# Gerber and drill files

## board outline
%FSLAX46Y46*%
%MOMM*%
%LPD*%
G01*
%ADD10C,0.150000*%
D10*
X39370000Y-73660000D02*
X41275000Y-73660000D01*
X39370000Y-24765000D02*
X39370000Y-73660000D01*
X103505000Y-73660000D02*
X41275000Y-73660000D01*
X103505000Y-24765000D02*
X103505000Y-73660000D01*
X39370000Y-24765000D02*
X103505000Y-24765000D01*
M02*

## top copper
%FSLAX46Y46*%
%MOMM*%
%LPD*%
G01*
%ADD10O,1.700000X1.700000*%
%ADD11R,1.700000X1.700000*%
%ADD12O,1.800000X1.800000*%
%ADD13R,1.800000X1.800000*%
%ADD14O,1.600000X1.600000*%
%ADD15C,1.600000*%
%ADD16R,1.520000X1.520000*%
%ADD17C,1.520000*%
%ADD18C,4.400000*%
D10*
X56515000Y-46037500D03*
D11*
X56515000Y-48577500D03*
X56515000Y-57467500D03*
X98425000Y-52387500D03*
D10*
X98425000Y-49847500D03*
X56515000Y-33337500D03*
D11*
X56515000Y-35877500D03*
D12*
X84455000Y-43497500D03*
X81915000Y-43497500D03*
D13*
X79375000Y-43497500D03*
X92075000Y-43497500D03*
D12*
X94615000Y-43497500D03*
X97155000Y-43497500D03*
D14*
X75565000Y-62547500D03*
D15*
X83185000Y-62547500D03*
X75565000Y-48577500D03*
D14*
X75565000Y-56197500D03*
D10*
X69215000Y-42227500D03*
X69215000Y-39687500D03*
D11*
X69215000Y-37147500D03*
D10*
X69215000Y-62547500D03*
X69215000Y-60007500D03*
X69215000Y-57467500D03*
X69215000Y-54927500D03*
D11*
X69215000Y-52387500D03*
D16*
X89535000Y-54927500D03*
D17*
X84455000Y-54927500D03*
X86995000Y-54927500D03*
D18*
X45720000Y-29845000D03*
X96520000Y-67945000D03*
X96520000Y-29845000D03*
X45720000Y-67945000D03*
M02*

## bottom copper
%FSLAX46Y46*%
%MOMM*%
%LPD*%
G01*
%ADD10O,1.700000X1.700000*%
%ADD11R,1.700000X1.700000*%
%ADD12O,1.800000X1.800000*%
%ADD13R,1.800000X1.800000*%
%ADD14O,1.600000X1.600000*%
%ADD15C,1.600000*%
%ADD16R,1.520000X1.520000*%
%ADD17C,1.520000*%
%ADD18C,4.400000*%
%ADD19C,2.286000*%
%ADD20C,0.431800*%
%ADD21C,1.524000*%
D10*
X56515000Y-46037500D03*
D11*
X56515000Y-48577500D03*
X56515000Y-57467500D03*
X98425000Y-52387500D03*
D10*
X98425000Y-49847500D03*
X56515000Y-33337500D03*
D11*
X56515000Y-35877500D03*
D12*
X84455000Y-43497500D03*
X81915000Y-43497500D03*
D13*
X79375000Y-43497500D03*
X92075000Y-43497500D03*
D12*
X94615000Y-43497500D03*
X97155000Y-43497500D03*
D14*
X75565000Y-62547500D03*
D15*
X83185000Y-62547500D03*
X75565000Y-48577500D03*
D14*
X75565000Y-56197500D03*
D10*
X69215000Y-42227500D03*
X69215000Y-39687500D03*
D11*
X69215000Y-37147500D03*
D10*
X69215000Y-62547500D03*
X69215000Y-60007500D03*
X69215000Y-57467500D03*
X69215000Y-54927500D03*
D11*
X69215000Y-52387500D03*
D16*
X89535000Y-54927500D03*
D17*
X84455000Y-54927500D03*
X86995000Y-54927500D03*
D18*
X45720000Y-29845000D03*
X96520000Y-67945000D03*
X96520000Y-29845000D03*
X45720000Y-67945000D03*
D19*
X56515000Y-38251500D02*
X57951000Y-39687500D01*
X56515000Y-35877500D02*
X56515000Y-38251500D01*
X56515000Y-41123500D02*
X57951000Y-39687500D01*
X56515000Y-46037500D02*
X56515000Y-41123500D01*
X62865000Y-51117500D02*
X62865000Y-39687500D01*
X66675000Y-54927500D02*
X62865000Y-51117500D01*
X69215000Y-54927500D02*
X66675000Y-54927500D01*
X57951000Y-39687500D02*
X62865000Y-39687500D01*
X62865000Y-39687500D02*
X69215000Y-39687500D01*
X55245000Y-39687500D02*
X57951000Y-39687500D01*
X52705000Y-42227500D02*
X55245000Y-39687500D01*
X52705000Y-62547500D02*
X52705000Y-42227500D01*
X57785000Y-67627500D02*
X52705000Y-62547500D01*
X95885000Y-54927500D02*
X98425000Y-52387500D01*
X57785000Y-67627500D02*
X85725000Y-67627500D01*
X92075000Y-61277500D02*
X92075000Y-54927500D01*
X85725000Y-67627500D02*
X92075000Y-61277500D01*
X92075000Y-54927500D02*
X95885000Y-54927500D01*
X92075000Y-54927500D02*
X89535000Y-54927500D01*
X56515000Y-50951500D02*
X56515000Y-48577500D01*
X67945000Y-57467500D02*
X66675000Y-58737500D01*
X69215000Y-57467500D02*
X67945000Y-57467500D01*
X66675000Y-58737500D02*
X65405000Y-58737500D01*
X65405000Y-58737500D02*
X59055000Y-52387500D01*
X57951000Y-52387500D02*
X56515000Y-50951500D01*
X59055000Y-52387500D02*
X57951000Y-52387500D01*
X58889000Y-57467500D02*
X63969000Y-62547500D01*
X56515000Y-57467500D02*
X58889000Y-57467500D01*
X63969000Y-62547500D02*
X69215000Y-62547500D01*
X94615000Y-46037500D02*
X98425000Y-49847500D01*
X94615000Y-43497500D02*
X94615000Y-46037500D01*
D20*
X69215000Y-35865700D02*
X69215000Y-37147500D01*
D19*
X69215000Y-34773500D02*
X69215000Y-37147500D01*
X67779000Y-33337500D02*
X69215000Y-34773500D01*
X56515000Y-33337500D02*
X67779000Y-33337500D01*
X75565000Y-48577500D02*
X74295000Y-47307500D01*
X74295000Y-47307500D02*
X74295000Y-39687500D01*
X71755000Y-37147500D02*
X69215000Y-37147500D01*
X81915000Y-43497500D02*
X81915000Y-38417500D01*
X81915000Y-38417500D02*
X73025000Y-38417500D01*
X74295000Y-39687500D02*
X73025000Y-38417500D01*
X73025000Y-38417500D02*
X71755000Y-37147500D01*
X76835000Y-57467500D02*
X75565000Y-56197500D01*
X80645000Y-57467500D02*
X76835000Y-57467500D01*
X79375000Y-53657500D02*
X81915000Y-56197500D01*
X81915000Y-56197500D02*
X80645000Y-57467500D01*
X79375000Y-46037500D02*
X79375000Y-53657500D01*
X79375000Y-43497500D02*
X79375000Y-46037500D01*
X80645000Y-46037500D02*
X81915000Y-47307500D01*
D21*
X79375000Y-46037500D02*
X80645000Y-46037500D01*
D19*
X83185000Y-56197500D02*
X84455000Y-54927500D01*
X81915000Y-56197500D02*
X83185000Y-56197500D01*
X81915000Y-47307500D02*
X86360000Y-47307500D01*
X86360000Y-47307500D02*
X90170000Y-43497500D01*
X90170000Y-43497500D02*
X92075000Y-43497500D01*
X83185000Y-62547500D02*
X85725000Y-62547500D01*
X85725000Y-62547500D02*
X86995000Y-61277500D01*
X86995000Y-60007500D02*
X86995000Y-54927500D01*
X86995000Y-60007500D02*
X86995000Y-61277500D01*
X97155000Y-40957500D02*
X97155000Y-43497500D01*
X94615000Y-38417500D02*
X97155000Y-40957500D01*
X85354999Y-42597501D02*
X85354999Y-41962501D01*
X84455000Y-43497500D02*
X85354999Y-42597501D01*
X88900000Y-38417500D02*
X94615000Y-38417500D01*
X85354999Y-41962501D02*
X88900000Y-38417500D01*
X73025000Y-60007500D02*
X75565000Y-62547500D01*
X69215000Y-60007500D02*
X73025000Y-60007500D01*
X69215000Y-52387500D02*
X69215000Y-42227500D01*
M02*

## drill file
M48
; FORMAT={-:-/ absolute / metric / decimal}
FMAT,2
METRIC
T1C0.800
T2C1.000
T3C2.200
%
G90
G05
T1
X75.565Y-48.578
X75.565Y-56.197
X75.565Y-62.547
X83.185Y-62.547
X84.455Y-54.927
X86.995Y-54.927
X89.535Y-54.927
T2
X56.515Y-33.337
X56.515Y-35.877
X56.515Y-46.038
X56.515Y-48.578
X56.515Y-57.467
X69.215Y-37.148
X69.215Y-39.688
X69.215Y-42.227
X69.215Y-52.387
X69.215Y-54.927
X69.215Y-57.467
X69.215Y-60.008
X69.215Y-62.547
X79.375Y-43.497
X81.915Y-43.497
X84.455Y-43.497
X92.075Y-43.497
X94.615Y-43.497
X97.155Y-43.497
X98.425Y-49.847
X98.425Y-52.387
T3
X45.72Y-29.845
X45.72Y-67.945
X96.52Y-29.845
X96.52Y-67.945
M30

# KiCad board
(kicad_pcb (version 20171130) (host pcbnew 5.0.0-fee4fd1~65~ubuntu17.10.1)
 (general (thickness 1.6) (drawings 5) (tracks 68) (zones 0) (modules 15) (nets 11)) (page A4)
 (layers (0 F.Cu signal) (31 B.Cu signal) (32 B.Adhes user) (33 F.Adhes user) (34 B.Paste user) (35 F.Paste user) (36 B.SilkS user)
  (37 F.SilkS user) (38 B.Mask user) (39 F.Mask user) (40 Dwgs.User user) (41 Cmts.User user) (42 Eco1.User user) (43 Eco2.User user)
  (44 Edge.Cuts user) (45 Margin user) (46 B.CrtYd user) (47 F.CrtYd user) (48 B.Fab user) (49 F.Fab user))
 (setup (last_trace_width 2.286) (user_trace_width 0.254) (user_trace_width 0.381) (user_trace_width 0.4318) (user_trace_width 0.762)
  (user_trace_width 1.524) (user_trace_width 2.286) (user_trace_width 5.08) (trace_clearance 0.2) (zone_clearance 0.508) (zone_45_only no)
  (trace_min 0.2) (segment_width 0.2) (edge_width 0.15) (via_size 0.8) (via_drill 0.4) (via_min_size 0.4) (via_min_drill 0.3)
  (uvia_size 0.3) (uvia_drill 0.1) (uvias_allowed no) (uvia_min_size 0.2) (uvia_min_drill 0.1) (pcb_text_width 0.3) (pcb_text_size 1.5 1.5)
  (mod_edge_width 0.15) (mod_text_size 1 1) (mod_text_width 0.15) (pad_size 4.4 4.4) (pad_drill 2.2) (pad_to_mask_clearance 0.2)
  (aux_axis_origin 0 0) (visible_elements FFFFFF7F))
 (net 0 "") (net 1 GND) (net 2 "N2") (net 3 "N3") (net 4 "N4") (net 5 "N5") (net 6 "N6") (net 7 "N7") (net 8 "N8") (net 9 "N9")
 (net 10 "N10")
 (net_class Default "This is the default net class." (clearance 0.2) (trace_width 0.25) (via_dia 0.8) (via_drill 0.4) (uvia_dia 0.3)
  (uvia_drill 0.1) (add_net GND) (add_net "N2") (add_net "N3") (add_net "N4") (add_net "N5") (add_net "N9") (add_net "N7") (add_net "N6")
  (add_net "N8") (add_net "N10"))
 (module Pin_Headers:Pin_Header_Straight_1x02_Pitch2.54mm (layer F.Cu) (at 56.515 48.5775 180)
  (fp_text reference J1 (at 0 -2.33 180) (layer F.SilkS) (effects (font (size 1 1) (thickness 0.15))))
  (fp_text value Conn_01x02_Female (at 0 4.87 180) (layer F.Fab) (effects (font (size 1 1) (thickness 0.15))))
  (pad 2 thru_hole oval (at 0 2.54 180) (size 1.7 1.7) (drill 1) (layers *.Cu *.Mask) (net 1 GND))
  (pad 1 thru_hole rect (at 0 0 180) (size 1.7 1.7) (drill 1) (layers *.Cu *.Mask) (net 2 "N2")))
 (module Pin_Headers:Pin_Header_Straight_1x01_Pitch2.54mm (layer F.Cu) (at 56.515 57.4675)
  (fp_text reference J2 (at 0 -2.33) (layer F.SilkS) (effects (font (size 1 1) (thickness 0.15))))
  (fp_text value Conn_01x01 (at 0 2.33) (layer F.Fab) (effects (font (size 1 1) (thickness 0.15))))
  (pad 1 thru_hole rect (at 0 0) (size 1.7 1.7) (drill 1) (layers *.Cu *.Mask) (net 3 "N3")))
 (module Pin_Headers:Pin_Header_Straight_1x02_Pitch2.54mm (layer F.Cu) (at 98.425 52.3875 180)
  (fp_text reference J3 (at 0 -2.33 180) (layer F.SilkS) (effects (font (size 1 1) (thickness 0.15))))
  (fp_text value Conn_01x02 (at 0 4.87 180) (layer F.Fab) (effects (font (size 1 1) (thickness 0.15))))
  (pad 1 thru_hole rect (at 0 0 180) (size 1.7 1.7) (drill 1) (layers *.Cu *.Mask) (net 1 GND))
  (pad 2 thru_hole oval (at 0 2.54 180) (size 1.7 1.7) (drill 1) (layers *.Cu *.Mask) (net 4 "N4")))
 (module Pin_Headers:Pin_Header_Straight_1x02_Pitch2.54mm (layer F.Cu) (at 56.515 35.8775 180)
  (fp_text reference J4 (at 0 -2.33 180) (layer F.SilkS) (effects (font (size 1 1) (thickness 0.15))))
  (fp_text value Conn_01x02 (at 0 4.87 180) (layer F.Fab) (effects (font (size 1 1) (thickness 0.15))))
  (pad 2 thru_hole oval (at 0 2.54 180) (size 1.7 1.7) (drill 1) (layers *.Cu *.Mask) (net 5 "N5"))
  (pad 1 thru_hole rect (at 0 0 180) (size 1.7 1.7) (drill 1) (layers *.Cu *.Mask) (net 1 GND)))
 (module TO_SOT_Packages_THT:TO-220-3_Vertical (layer F.Cu) (at 79.375 43.4975)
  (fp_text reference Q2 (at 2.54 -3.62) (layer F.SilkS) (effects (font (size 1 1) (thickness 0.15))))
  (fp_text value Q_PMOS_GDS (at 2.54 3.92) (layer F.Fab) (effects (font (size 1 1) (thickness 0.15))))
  (pad 3 thru_hole oval (at 5.08 0) (size 1.8 1.8) (drill 1) (layers *.Cu *.Mask) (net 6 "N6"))
  (pad 2 thru_hole oval (at 2.54 0) (size 1.8 1.8) (drill 1) (layers *.Cu *.Mask) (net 5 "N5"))
  (pad 1 thru_hole rect (at 0 0) (size 1.8 1.8) (drill 1) (layers *.Cu *.Mask) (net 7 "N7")))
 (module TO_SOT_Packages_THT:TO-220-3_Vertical (layer F.Cu) (at 92.075 43.4975)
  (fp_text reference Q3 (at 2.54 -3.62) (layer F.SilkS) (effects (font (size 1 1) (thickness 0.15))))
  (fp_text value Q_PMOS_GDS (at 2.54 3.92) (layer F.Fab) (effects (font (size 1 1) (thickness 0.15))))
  (pad 1 thru_hole rect (at 0 0) (size 1.8 1.8) (drill 1) (layers *.Cu *.Mask) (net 7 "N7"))
  (pad 2 thru_hole oval (at 2.54 0) (size 1.8 1.8) (drill 1) (layers *.Cu *.Mask) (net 4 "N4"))
  (pad 3 thru_hole oval (at 5.08 0) (size 1.8 1.8) (drill 1) (layers *.Cu *.Mask) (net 6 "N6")))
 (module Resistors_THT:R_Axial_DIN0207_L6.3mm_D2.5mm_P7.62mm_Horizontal (layer F.Cu) (at 83.185 62.5475 180)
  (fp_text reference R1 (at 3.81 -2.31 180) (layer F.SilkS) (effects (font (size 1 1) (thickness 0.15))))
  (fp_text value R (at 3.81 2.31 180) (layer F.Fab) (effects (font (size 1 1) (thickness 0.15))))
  (pad 2 thru_hole oval (at 7.62 0 180) (size 1.6 1.6) (drill 0.8) (layers *.Cu *.Mask) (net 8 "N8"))
  (pad 1 thru_hole circle (at 0 0 180) (size 1.6 1.6) (drill 0.8) (layers *.Cu *.Mask) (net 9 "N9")))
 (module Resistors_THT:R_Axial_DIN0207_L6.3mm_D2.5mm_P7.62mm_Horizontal (layer F.Cu) (at 75.565 48.5775 270)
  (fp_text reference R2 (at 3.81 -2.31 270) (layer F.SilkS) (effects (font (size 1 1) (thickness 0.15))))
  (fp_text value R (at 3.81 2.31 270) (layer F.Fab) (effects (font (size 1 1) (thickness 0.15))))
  (pad 1 thru_hole circle (at 0 0 270) (size 1.6 1.6) (drill 0.8) (layers *.Cu *.Mask) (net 5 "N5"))
  (pad 2 thru_hole oval (at 7.62 0 270) (size 1.6 1.6) (drill 0.8) (layers *.Cu *.Mask) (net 7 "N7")))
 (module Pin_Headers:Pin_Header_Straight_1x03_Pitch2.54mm (layer F.Cu) (at 69.215 37.1475)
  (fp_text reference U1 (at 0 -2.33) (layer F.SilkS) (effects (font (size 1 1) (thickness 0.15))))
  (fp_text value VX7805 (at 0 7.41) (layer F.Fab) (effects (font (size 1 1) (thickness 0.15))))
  (pad 3 thru_hole oval (at 0 5.08) (size 1.7 1.7) (drill 1) (layers *.Cu *.Mask) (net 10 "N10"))
  (pad 2 thru_hole oval (at 0 2.54) (size 1.7 1.7) (drill 1) (layers *.Cu *.Mask) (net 1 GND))
  (pad 1 thru_hole rect (at 0 0) (size 1.7 1.7) (drill 1) (layers *.Cu *.Mask) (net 5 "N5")))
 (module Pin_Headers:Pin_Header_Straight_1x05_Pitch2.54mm (layer F.Cu) (at 69.215 52.3875)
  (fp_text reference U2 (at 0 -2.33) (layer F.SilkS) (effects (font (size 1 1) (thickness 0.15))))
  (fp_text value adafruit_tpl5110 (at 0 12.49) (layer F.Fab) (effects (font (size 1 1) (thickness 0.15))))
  (pad 5 thru_hole oval (at 0 10.16) (size 1.7 1.7) (drill 1) (layers *.Cu *.Mask) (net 3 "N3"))
  (pad 4 thru_hole oval (at 0 7.62) (size 1.7 1.7) (drill 1) (layers *.Cu *.Mask) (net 8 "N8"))
  (pad 3 thru_hole oval (at 0 5.08) (size 1.7 1.7) (drill 1) (layers *.Cu *.Mask) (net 2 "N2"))
  (pad 2 thru_hole oval (at 0 2.54) (size 1.7 1.7) (drill 1) (layers *.Cu *.Mask) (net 1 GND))
  (pad 1 thru_hole rect (at 0 0) (size 1.7 1.7) (drill 1) (layers *.Cu *.Mask) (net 10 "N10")))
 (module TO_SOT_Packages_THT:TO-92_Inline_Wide (layer F.Cu) (at 89.535 54.9275 180)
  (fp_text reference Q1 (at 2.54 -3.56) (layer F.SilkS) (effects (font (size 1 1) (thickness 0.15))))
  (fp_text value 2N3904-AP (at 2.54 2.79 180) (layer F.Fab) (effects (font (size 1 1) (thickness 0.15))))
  (pad 1 thru_hole rect (at 0 0 270) (size 1.52 1.52) (drill 0.8) (layers *.Cu *.Mask) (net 1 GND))
  (pad 3 thru_hole circle (at 5.08 0 270) (size 1.52 1.52) (drill 0.8) (layers *.Cu *.Mask) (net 7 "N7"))
  (pad 2 thru_hole circle (at 2.54 0 270) (size 1.52 1.52) (drill 0.8) (layers *.Cu *.Mask) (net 9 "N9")))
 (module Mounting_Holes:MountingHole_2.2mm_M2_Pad (layer F.Cu) (at 45.72 29.845)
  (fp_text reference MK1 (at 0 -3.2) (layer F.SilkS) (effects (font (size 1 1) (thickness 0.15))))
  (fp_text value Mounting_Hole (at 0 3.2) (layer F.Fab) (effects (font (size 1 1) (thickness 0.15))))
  (pad 1 thru_hole circle (at 0 0) (size 4.4 4.4) (drill 2.2) (layers *.Cu *.Mask)))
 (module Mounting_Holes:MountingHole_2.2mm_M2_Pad (layer F.Cu) (at 96.52 67.945)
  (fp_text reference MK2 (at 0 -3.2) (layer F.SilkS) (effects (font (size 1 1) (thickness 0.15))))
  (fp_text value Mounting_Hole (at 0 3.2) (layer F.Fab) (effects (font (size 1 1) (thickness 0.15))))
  (pad 1 thru_hole circle (at 0 0) (size 4.4 4.4) (drill 2.2) (layers *.Cu *.Mask)))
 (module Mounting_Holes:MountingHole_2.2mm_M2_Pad (layer F.Cu) (at 96.52 29.845)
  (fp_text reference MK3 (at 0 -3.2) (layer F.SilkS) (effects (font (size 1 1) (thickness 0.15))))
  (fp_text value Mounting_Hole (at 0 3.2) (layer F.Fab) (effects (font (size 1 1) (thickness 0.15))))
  (pad 1 thru_hole circle (at 0 0) (size 4.4 4.4) (drill 2.2) (layers *.Cu *.Mask)))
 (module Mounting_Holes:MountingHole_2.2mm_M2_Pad (layer F.Cu) (at 45.72 67.945)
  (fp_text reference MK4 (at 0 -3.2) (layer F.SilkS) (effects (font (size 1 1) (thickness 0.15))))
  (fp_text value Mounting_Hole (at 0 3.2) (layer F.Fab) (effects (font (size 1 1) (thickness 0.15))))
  (pad 1 thru_hole circle (at 0 0) (size 4.4 4.4) (drill 2.2) (layers *.Cu *.Mask)))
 (gr_line (start 39.37 73.66) (end 41.275 73.66) (layer Edge.Cuts) (width 0.15))
 (gr_line (start 39.37 24.765) (end 39.37 73.66) (layer Edge.Cuts) (width 0.15))
 (gr_line (start 103.505 73.66) (end 41.275 73.66) (layer Edge.Cuts) (width 0.15))
 (gr_line (start 103.505 24.765) (end 103.505 73.66) (layer Edge.Cuts) (width 0.15))
 (gr_line (start 39.37 24.765) (end 103.505 24.765) (layer Edge.Cuts) (width 0.15))
 (segment (start 56.515 38.2515) (end 57.951 39.6875) (width 2.286) (layer B.Cu) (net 1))
 (segment (start 56.515 35.8775) (end 56.515 38.2515) (width 2.286) (layer B.Cu) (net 1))
 (segment (start 56.515 41.1235) (end 57.951 39.6875) (width 2.286) (layer B.Cu) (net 1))
 (segment (start 56.515 46.0375) (end 56.515 41.1235) (width 2.286) (layer B.Cu) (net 1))
 (segment (start 62.865 51.1175) (end 62.865 39.6875) (width 2.286) (layer B.Cu) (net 1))
 (segment (start 66.675 54.9275) (end 62.865 51.1175) (width 2.286) (layer B.Cu) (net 1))
 (segment (start 69.215 54.9275) (end 66.675 54.9275) (width 2.286) (layer B.Cu) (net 1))
 (segment (start 57.951 39.6875) (end 62.865 39.6875) (width 2.286) (layer B.Cu) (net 1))
 (segment (start 62.865 39.6875) (end 69.215 39.6875) (width 2.286) (layer B.Cu) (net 1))
 (segment (start 55.245 39.6875) (end 57.951 39.6875) (width 2.286) (layer B.Cu) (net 1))
 (segment (start 52.705 42.2275) (end 55.245 39.6875) (width 2.286) (layer B.Cu) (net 1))
 (segment (start 52.705 62.5475) (end 52.705 42.2275) (width 2.286) (layer B.Cu) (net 1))
 (segment (start 57.785 67.6275) (end 52.705 62.5475) (width 2.286) (layer B.Cu) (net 1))
 (segment (start 95.885 54.9275) (end 98.425 52.3875) (width 2.286) (layer B.Cu) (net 1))
 (segment (start 57.785 67.6275) (end 85.725 67.6275) (width 2.286) (layer B.Cu) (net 1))
 (segment (start 92.075 61.2775) (end 92.075 54.9275) (width 2.286) (layer B.Cu) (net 1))
 (segment (start 85.725 67.6275) (end 92.075 61.2775) (width 2.286) (layer B.Cu) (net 1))
 (segment (start 92.075 54.9275) (end 95.885 54.9275) (width 2.286) (layer B.Cu) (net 1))
 (segment (start 92.075 54.9275) (end 89.535 54.9275) (width 2.286) (layer B.Cu) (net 1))
 (segment (start 56.515 50.9515) (end 56.515 48.5775) (width 2.286) (layer B.Cu) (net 2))
 (segment (start 67.945 57.4675) (end 66.675 58.7375) (width 2.286) (layer B.Cu) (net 2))
 (segment (start 69.215 57.4675) (end 67.945 57.4675) (width 2.286) (layer B.Cu) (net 2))
 (segment (start 66.675 58.7375) (end 65.405 58.7375) (width 2.286) (layer B.Cu) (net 2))
 (segment (start 65.405 58.7375) (end 59.055 52.3875) (width 2.286) (layer B.Cu) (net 2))
 (segment (start 57.951 52.3875) (end 56.515 50.9515) (width 2.286) (layer B.Cu) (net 2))
 (segment (start 59.055 52.3875) (end 57.951 52.3875) (width 2.286) (layer B.Cu) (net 2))
 (segment (start 58.889 57.4675) (end 63.969 62.5475) (width 2.286) (layer B.Cu) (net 3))
 (segment (start 56.515 57.4675) (end 58.889 57.4675) (width 2.286) (layer B.Cu) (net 3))
 (segment (start 63.969 62.5475) (end 69.215 62.5475) (width 2.286) (layer B.Cu) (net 3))
 (segment (start 94.615 46.0375) (end 98.425 49.8475) (width 2.286) (layer B.Cu) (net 4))
 (segment (start 94.615 43.4975) (end 94.615 46.0375) (width 2.286) (layer B.Cu) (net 4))
 (segment (start 69.215 35.8657) (end 69.215 37.1475) (width 0.4318) (layer B.Cu) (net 5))
 (segment (start 69.215 34.7735) (end 69.215 37.1475) (width 2.286) (layer B.Cu) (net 5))
 (segment (start 67.779 33.3375) (end 69.215 34.7735) (width 2.286) (layer B.Cu) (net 5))
 (segment (start 56.515 33.3375) (end 67.779 33.3375) (width 2.286) (layer B.Cu) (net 5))
 (segment (start 75.565 48.5775) (end 74.295 47.3075) (width 2.286) (layer B.Cu) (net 5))
 (segment (start 74.295 47.3075) (end 74.295 39.6875) (width 2.286) (layer B.Cu) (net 5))
 (segment (start 71.755 37.1475) (end 69.215 37.1475) (width 2.286) (layer B.Cu) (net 5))
 (segment (start 81.915 43.4975) (end 81.915 38.4175) (width 2.286) (layer B.Cu) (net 5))
 (segment (start 81.915 38.4175) (end 73.025 38.4175) (width 2.286) (layer B.Cu) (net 5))
 (segment (start 74.295 39.6875) (end 73.025 38.4175) (width 2.286) (layer B.Cu) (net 5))
 (segment (start 73.025 38.4175) (end 71.755 37.1475) (width 2.286) (layer B.Cu) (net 5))
 (segment (start 76.835 57.4675) (end 75.565 56.1975) (width 2.286) (layer B.Cu) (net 7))
 (segment (start 80.645 57.4675) (end 76.835 57.4675) (width 2.286) (layer B.Cu) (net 7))
 (segment (start 79.375 53.6575) (end 81.915 56.1975) (width 2.286) (layer B.Cu) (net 7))
 (segment (start 81.915 56.1975) (end 80.645 57.4675) (width 2.286) (layer B.Cu) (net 7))
 (segment (start 79.375 46.0375) (end 79.375 53.6575) (width 2.286) (layer B.Cu) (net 7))
 (segment (start 79.375 43.4975) (end 79.375 46.0375) (width 2.286) (layer B.Cu) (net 7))
 (segment (start 80.645 46.0375) (end 81.915 47.3075) (width 2.286) (layer B.Cu) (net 7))
 (segment (start 79.375 46.0375) (end 80.645 46.0375) (width 1.524) (layer B.Cu) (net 7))
 (segment (start 83.185 56.1975) (end 84.455 54.9275) (width 2.286) (layer B.Cu) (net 7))
 (segment (start 81.915 56.1975) (end 83.185 56.1975) (width 2.286) (layer B.Cu) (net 7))
 (segment (start 81.915 47.3075) (end 86.36 47.3075) (width 2.286) (layer B.Cu) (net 7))
 (segment (start 86.36 47.3075) (end 90.17 43.4975) (width 2.286) (layer B.Cu) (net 7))
 (segment (start 90.17 43.4975) (end 92.075 43.4975) (width 2.286) (layer B.Cu) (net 7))
 (segment (start 83.185 62.5475) (end 85.725 62.5475) (width 2.286) (layer B.Cu) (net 9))
 (segment (start 85.725 62.5475) (end 86.995 61.2775) (width 2.286) (layer B.Cu) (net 9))
 (segment (start 86.995 60.0075) (end 86.995 54.9275) (width 2.286) (layer B.Cu) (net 9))
 (segment (start 86.995 60.0075) (end 86.995 61.2775) (width 2.286) (layer B.Cu) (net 9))
 (segment (start 97.155 40.9575) (end 97.155 43.4975) (width 2.286) (layer B.Cu) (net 6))
 (segment (start 94.615 38.4175) (end 97.155 40.9575) (width 2.286) (layer B.Cu) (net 6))
 (segment (start 85.354999 42.597501) (end 85.354999 41.962501) (width 2.286) (layer B.Cu) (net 6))
 (segment (start 84.455 43.4975) (end 85.354999 42.597501) (width 2.286) (layer B.Cu) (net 6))
 (segment (start 88.9 38.4175) (end 94.615 38.4175) (width 2.286) (layer B.Cu) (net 6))
 (segment (start 85.354999 41.962501) (end 88.9 38.4175) (width 2.286) (layer B.Cu) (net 6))
 (segment (start 73.025 60.0075) (end 75.565 62.5475) (width 2.286) (layer B.Cu) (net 8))
 (segment (start 69.215 60.0075) (end 73.025 60.0075) (width 2.286) (layer B.Cu) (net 8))
 (segment (start 69.215 52.3875) (end 69.215 42.2275) (width 2.286) (layer B.Cu) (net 10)))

